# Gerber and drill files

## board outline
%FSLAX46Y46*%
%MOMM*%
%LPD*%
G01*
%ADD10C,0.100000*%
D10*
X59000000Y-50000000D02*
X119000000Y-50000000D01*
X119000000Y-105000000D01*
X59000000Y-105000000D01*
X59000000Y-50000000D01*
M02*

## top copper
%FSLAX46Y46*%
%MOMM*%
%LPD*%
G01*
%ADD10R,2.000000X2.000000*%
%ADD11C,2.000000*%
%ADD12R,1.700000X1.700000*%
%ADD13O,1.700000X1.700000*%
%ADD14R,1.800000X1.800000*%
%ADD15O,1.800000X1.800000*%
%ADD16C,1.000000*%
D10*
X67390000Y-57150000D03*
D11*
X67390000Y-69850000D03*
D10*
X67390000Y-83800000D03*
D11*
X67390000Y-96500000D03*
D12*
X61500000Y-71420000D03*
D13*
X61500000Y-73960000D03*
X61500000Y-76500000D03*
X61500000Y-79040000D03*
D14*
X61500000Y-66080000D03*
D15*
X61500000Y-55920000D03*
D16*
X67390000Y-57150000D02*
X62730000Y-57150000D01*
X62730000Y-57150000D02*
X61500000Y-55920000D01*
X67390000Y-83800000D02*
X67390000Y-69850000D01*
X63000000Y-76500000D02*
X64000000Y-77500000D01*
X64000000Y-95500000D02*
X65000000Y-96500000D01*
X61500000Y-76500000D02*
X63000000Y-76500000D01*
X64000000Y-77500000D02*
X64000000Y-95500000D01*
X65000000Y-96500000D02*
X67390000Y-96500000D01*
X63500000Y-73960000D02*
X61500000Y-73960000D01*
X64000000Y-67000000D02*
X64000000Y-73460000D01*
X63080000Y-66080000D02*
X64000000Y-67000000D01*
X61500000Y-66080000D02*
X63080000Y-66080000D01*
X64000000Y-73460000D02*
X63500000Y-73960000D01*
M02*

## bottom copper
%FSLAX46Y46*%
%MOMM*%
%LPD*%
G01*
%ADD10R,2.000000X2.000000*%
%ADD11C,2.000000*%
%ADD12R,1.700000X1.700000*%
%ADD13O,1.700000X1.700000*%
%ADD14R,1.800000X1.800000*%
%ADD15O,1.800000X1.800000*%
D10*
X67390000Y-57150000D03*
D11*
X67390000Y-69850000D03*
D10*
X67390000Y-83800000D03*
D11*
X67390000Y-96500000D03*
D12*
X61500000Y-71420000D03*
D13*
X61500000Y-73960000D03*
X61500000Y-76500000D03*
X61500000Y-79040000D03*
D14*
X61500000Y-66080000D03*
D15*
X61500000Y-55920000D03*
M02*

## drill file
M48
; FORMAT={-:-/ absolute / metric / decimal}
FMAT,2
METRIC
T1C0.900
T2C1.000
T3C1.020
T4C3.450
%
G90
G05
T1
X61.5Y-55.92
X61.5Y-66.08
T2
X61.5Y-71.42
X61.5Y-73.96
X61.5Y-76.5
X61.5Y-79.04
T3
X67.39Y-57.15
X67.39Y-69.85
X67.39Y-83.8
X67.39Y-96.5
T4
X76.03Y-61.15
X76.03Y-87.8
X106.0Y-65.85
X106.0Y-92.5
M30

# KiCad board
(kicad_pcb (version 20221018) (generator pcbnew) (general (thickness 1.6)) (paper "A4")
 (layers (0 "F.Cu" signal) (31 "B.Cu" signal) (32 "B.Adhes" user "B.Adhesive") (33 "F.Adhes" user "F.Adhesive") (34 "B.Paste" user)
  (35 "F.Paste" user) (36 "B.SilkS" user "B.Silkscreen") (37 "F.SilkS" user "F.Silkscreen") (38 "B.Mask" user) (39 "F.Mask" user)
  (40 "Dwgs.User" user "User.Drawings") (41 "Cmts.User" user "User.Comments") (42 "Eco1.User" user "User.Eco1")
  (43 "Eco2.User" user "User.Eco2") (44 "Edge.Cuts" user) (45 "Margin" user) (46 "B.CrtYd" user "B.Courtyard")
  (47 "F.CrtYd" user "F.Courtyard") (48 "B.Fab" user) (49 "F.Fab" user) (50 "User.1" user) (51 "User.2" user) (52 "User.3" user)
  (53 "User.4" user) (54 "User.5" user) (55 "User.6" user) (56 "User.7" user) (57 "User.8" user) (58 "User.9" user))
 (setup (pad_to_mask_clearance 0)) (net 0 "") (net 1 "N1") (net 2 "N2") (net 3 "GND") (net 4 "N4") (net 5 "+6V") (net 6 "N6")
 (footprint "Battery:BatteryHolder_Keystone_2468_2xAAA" (layer "F.Cu") (at 67.39 57.15)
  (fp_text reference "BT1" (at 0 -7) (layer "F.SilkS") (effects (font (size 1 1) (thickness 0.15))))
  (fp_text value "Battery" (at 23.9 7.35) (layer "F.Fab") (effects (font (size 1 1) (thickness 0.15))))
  (pad "" np_thru_hole circle (at 8.64 4) (size 3.45 3.45) (drill 3.45) (layers "*.Cu"))
  (pad "" np_thru_hole circle (at 38.61 8.7) (size 3.45 3.45) (drill 3.45) (layers "*.Cu" "*.Mask"))
  (pad "1" thru_hole rect (at 0 0) (size 2 2) (drill 1.02) (layers "*.Cu" "*.Mask") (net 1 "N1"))
  (pad "2" thru_hole circle (at 0 12.7) (size 2 2) (drill 1.02) (layers "*.Cu" "*.Mask") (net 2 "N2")))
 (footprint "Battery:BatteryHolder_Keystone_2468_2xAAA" (layer "F.Cu") (at 67.39 83.8)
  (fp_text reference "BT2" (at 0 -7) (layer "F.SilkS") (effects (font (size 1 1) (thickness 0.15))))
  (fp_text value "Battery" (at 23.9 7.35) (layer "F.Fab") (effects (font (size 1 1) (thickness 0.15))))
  (pad "" np_thru_hole circle (at 8.64 4) (size 3.45 3.45) (drill 3.45) (layers "*.Cu"))
  (pad "" np_thru_hole circle (at 38.61 8.7) (size 3.45 3.45) (drill 3.45) (layers "*.Cu" "*.Mask"))
  (pad "1" thru_hole rect (at 0 0) (size 2 2) (drill 1.02) (layers "*.Cu" "*.Mask") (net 2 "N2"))
  (pad "2" thru_hole circle (at 0 12.7) (size 2 2) (drill 1.02) (layers "*.Cu" "*.Mask") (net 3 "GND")))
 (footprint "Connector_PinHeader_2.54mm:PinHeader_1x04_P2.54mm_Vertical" (layer "F.Cu") (at 61.5 71.42)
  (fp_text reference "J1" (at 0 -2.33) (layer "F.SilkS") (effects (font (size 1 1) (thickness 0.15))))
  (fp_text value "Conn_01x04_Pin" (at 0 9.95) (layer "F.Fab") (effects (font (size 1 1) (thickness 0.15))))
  (pad "1" thru_hole rect (at 0 0) (size 1.7 1.7) (drill 1) (layers "*.Cu" "*.Mask") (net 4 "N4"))
  (pad "2" thru_hole oval (at 0 2.54) (size 1.7 1.7) (drill 1) (layers "*.Cu" "*.Mask") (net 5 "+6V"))
  (pad "3" thru_hole oval (at 0 5.08) (size 1.7 1.7) (drill 1) (layers "*.Cu" "*.Mask") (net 3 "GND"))
  (pad "4" thru_hole oval (at 0 7.62) (size 1.7 1.7) (drill 1) (layers "*.Cu" "*.Mask") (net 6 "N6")))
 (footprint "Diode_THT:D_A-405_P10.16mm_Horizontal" (layer "F.Cu") (at 61.5 66.08 90)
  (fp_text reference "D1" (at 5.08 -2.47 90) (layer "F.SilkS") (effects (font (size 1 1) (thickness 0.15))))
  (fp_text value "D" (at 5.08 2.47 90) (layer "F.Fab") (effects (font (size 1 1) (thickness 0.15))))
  (pad "1" thru_hole rect (at 0 0 90) (size 1.8 1.8) (drill 0.9) (layers "*.Cu" "*.Mask") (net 5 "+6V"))
  (pad "2" thru_hole oval (at 10.16 0 90) (size 1.8 1.8) (drill 0.9) (layers "*.Cu" "*.Mask") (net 1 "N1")))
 (gr_rect (start 59 50) (end 119 105) (stroke (width 0.1) (type default)) (fill none) (layer "Edge.Cuts"))
 (segment (start 67.39 57.15) (end 62.73 57.15) (width 1) (layer "F.Cu") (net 1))
 (segment (start 62.73 57.15) (end 61.5 55.92) (width 1) (layer "F.Cu") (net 1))
 (segment (start 67.39 83.8) (end 67.39 69.85) (width 1) (layer "F.Cu") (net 2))
 (segment (start 63 76.5) (end 64 77.5) (width 1) (layer "F.Cu") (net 3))
 (segment (start 64 95.5) (end 65 96.5) (width 1) (layer "F.Cu") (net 3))
 (segment (start 61.5 76.5) (end 63 76.5) (width 1) (layer "F.Cu") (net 3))
 (segment (start 64 77.5) (end 64 95.5) (width 1) (layer "F.Cu") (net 3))
 (segment (start 65 96.5) (end 67.39 96.5) (width 1) (layer "F.Cu") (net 3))
 (segment (start 63.5 73.96) (end 61.5 73.96) (width 1) (layer "F.Cu") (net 5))
 (segment (start 64 67) (end 64 73.46) (width 1) (layer "F.Cu") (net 5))
 (segment (start 63.08 66.08) (end 64 67) (width 1) (layer "F.Cu") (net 5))
 (segment (start 61.5 66.08) (end 63.08 66.08) (width 1) (layer "F.Cu") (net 5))
 (segment (start 64 73.46) (end 63.5 73.96) (width 1) (layer "F.Cu") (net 5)))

